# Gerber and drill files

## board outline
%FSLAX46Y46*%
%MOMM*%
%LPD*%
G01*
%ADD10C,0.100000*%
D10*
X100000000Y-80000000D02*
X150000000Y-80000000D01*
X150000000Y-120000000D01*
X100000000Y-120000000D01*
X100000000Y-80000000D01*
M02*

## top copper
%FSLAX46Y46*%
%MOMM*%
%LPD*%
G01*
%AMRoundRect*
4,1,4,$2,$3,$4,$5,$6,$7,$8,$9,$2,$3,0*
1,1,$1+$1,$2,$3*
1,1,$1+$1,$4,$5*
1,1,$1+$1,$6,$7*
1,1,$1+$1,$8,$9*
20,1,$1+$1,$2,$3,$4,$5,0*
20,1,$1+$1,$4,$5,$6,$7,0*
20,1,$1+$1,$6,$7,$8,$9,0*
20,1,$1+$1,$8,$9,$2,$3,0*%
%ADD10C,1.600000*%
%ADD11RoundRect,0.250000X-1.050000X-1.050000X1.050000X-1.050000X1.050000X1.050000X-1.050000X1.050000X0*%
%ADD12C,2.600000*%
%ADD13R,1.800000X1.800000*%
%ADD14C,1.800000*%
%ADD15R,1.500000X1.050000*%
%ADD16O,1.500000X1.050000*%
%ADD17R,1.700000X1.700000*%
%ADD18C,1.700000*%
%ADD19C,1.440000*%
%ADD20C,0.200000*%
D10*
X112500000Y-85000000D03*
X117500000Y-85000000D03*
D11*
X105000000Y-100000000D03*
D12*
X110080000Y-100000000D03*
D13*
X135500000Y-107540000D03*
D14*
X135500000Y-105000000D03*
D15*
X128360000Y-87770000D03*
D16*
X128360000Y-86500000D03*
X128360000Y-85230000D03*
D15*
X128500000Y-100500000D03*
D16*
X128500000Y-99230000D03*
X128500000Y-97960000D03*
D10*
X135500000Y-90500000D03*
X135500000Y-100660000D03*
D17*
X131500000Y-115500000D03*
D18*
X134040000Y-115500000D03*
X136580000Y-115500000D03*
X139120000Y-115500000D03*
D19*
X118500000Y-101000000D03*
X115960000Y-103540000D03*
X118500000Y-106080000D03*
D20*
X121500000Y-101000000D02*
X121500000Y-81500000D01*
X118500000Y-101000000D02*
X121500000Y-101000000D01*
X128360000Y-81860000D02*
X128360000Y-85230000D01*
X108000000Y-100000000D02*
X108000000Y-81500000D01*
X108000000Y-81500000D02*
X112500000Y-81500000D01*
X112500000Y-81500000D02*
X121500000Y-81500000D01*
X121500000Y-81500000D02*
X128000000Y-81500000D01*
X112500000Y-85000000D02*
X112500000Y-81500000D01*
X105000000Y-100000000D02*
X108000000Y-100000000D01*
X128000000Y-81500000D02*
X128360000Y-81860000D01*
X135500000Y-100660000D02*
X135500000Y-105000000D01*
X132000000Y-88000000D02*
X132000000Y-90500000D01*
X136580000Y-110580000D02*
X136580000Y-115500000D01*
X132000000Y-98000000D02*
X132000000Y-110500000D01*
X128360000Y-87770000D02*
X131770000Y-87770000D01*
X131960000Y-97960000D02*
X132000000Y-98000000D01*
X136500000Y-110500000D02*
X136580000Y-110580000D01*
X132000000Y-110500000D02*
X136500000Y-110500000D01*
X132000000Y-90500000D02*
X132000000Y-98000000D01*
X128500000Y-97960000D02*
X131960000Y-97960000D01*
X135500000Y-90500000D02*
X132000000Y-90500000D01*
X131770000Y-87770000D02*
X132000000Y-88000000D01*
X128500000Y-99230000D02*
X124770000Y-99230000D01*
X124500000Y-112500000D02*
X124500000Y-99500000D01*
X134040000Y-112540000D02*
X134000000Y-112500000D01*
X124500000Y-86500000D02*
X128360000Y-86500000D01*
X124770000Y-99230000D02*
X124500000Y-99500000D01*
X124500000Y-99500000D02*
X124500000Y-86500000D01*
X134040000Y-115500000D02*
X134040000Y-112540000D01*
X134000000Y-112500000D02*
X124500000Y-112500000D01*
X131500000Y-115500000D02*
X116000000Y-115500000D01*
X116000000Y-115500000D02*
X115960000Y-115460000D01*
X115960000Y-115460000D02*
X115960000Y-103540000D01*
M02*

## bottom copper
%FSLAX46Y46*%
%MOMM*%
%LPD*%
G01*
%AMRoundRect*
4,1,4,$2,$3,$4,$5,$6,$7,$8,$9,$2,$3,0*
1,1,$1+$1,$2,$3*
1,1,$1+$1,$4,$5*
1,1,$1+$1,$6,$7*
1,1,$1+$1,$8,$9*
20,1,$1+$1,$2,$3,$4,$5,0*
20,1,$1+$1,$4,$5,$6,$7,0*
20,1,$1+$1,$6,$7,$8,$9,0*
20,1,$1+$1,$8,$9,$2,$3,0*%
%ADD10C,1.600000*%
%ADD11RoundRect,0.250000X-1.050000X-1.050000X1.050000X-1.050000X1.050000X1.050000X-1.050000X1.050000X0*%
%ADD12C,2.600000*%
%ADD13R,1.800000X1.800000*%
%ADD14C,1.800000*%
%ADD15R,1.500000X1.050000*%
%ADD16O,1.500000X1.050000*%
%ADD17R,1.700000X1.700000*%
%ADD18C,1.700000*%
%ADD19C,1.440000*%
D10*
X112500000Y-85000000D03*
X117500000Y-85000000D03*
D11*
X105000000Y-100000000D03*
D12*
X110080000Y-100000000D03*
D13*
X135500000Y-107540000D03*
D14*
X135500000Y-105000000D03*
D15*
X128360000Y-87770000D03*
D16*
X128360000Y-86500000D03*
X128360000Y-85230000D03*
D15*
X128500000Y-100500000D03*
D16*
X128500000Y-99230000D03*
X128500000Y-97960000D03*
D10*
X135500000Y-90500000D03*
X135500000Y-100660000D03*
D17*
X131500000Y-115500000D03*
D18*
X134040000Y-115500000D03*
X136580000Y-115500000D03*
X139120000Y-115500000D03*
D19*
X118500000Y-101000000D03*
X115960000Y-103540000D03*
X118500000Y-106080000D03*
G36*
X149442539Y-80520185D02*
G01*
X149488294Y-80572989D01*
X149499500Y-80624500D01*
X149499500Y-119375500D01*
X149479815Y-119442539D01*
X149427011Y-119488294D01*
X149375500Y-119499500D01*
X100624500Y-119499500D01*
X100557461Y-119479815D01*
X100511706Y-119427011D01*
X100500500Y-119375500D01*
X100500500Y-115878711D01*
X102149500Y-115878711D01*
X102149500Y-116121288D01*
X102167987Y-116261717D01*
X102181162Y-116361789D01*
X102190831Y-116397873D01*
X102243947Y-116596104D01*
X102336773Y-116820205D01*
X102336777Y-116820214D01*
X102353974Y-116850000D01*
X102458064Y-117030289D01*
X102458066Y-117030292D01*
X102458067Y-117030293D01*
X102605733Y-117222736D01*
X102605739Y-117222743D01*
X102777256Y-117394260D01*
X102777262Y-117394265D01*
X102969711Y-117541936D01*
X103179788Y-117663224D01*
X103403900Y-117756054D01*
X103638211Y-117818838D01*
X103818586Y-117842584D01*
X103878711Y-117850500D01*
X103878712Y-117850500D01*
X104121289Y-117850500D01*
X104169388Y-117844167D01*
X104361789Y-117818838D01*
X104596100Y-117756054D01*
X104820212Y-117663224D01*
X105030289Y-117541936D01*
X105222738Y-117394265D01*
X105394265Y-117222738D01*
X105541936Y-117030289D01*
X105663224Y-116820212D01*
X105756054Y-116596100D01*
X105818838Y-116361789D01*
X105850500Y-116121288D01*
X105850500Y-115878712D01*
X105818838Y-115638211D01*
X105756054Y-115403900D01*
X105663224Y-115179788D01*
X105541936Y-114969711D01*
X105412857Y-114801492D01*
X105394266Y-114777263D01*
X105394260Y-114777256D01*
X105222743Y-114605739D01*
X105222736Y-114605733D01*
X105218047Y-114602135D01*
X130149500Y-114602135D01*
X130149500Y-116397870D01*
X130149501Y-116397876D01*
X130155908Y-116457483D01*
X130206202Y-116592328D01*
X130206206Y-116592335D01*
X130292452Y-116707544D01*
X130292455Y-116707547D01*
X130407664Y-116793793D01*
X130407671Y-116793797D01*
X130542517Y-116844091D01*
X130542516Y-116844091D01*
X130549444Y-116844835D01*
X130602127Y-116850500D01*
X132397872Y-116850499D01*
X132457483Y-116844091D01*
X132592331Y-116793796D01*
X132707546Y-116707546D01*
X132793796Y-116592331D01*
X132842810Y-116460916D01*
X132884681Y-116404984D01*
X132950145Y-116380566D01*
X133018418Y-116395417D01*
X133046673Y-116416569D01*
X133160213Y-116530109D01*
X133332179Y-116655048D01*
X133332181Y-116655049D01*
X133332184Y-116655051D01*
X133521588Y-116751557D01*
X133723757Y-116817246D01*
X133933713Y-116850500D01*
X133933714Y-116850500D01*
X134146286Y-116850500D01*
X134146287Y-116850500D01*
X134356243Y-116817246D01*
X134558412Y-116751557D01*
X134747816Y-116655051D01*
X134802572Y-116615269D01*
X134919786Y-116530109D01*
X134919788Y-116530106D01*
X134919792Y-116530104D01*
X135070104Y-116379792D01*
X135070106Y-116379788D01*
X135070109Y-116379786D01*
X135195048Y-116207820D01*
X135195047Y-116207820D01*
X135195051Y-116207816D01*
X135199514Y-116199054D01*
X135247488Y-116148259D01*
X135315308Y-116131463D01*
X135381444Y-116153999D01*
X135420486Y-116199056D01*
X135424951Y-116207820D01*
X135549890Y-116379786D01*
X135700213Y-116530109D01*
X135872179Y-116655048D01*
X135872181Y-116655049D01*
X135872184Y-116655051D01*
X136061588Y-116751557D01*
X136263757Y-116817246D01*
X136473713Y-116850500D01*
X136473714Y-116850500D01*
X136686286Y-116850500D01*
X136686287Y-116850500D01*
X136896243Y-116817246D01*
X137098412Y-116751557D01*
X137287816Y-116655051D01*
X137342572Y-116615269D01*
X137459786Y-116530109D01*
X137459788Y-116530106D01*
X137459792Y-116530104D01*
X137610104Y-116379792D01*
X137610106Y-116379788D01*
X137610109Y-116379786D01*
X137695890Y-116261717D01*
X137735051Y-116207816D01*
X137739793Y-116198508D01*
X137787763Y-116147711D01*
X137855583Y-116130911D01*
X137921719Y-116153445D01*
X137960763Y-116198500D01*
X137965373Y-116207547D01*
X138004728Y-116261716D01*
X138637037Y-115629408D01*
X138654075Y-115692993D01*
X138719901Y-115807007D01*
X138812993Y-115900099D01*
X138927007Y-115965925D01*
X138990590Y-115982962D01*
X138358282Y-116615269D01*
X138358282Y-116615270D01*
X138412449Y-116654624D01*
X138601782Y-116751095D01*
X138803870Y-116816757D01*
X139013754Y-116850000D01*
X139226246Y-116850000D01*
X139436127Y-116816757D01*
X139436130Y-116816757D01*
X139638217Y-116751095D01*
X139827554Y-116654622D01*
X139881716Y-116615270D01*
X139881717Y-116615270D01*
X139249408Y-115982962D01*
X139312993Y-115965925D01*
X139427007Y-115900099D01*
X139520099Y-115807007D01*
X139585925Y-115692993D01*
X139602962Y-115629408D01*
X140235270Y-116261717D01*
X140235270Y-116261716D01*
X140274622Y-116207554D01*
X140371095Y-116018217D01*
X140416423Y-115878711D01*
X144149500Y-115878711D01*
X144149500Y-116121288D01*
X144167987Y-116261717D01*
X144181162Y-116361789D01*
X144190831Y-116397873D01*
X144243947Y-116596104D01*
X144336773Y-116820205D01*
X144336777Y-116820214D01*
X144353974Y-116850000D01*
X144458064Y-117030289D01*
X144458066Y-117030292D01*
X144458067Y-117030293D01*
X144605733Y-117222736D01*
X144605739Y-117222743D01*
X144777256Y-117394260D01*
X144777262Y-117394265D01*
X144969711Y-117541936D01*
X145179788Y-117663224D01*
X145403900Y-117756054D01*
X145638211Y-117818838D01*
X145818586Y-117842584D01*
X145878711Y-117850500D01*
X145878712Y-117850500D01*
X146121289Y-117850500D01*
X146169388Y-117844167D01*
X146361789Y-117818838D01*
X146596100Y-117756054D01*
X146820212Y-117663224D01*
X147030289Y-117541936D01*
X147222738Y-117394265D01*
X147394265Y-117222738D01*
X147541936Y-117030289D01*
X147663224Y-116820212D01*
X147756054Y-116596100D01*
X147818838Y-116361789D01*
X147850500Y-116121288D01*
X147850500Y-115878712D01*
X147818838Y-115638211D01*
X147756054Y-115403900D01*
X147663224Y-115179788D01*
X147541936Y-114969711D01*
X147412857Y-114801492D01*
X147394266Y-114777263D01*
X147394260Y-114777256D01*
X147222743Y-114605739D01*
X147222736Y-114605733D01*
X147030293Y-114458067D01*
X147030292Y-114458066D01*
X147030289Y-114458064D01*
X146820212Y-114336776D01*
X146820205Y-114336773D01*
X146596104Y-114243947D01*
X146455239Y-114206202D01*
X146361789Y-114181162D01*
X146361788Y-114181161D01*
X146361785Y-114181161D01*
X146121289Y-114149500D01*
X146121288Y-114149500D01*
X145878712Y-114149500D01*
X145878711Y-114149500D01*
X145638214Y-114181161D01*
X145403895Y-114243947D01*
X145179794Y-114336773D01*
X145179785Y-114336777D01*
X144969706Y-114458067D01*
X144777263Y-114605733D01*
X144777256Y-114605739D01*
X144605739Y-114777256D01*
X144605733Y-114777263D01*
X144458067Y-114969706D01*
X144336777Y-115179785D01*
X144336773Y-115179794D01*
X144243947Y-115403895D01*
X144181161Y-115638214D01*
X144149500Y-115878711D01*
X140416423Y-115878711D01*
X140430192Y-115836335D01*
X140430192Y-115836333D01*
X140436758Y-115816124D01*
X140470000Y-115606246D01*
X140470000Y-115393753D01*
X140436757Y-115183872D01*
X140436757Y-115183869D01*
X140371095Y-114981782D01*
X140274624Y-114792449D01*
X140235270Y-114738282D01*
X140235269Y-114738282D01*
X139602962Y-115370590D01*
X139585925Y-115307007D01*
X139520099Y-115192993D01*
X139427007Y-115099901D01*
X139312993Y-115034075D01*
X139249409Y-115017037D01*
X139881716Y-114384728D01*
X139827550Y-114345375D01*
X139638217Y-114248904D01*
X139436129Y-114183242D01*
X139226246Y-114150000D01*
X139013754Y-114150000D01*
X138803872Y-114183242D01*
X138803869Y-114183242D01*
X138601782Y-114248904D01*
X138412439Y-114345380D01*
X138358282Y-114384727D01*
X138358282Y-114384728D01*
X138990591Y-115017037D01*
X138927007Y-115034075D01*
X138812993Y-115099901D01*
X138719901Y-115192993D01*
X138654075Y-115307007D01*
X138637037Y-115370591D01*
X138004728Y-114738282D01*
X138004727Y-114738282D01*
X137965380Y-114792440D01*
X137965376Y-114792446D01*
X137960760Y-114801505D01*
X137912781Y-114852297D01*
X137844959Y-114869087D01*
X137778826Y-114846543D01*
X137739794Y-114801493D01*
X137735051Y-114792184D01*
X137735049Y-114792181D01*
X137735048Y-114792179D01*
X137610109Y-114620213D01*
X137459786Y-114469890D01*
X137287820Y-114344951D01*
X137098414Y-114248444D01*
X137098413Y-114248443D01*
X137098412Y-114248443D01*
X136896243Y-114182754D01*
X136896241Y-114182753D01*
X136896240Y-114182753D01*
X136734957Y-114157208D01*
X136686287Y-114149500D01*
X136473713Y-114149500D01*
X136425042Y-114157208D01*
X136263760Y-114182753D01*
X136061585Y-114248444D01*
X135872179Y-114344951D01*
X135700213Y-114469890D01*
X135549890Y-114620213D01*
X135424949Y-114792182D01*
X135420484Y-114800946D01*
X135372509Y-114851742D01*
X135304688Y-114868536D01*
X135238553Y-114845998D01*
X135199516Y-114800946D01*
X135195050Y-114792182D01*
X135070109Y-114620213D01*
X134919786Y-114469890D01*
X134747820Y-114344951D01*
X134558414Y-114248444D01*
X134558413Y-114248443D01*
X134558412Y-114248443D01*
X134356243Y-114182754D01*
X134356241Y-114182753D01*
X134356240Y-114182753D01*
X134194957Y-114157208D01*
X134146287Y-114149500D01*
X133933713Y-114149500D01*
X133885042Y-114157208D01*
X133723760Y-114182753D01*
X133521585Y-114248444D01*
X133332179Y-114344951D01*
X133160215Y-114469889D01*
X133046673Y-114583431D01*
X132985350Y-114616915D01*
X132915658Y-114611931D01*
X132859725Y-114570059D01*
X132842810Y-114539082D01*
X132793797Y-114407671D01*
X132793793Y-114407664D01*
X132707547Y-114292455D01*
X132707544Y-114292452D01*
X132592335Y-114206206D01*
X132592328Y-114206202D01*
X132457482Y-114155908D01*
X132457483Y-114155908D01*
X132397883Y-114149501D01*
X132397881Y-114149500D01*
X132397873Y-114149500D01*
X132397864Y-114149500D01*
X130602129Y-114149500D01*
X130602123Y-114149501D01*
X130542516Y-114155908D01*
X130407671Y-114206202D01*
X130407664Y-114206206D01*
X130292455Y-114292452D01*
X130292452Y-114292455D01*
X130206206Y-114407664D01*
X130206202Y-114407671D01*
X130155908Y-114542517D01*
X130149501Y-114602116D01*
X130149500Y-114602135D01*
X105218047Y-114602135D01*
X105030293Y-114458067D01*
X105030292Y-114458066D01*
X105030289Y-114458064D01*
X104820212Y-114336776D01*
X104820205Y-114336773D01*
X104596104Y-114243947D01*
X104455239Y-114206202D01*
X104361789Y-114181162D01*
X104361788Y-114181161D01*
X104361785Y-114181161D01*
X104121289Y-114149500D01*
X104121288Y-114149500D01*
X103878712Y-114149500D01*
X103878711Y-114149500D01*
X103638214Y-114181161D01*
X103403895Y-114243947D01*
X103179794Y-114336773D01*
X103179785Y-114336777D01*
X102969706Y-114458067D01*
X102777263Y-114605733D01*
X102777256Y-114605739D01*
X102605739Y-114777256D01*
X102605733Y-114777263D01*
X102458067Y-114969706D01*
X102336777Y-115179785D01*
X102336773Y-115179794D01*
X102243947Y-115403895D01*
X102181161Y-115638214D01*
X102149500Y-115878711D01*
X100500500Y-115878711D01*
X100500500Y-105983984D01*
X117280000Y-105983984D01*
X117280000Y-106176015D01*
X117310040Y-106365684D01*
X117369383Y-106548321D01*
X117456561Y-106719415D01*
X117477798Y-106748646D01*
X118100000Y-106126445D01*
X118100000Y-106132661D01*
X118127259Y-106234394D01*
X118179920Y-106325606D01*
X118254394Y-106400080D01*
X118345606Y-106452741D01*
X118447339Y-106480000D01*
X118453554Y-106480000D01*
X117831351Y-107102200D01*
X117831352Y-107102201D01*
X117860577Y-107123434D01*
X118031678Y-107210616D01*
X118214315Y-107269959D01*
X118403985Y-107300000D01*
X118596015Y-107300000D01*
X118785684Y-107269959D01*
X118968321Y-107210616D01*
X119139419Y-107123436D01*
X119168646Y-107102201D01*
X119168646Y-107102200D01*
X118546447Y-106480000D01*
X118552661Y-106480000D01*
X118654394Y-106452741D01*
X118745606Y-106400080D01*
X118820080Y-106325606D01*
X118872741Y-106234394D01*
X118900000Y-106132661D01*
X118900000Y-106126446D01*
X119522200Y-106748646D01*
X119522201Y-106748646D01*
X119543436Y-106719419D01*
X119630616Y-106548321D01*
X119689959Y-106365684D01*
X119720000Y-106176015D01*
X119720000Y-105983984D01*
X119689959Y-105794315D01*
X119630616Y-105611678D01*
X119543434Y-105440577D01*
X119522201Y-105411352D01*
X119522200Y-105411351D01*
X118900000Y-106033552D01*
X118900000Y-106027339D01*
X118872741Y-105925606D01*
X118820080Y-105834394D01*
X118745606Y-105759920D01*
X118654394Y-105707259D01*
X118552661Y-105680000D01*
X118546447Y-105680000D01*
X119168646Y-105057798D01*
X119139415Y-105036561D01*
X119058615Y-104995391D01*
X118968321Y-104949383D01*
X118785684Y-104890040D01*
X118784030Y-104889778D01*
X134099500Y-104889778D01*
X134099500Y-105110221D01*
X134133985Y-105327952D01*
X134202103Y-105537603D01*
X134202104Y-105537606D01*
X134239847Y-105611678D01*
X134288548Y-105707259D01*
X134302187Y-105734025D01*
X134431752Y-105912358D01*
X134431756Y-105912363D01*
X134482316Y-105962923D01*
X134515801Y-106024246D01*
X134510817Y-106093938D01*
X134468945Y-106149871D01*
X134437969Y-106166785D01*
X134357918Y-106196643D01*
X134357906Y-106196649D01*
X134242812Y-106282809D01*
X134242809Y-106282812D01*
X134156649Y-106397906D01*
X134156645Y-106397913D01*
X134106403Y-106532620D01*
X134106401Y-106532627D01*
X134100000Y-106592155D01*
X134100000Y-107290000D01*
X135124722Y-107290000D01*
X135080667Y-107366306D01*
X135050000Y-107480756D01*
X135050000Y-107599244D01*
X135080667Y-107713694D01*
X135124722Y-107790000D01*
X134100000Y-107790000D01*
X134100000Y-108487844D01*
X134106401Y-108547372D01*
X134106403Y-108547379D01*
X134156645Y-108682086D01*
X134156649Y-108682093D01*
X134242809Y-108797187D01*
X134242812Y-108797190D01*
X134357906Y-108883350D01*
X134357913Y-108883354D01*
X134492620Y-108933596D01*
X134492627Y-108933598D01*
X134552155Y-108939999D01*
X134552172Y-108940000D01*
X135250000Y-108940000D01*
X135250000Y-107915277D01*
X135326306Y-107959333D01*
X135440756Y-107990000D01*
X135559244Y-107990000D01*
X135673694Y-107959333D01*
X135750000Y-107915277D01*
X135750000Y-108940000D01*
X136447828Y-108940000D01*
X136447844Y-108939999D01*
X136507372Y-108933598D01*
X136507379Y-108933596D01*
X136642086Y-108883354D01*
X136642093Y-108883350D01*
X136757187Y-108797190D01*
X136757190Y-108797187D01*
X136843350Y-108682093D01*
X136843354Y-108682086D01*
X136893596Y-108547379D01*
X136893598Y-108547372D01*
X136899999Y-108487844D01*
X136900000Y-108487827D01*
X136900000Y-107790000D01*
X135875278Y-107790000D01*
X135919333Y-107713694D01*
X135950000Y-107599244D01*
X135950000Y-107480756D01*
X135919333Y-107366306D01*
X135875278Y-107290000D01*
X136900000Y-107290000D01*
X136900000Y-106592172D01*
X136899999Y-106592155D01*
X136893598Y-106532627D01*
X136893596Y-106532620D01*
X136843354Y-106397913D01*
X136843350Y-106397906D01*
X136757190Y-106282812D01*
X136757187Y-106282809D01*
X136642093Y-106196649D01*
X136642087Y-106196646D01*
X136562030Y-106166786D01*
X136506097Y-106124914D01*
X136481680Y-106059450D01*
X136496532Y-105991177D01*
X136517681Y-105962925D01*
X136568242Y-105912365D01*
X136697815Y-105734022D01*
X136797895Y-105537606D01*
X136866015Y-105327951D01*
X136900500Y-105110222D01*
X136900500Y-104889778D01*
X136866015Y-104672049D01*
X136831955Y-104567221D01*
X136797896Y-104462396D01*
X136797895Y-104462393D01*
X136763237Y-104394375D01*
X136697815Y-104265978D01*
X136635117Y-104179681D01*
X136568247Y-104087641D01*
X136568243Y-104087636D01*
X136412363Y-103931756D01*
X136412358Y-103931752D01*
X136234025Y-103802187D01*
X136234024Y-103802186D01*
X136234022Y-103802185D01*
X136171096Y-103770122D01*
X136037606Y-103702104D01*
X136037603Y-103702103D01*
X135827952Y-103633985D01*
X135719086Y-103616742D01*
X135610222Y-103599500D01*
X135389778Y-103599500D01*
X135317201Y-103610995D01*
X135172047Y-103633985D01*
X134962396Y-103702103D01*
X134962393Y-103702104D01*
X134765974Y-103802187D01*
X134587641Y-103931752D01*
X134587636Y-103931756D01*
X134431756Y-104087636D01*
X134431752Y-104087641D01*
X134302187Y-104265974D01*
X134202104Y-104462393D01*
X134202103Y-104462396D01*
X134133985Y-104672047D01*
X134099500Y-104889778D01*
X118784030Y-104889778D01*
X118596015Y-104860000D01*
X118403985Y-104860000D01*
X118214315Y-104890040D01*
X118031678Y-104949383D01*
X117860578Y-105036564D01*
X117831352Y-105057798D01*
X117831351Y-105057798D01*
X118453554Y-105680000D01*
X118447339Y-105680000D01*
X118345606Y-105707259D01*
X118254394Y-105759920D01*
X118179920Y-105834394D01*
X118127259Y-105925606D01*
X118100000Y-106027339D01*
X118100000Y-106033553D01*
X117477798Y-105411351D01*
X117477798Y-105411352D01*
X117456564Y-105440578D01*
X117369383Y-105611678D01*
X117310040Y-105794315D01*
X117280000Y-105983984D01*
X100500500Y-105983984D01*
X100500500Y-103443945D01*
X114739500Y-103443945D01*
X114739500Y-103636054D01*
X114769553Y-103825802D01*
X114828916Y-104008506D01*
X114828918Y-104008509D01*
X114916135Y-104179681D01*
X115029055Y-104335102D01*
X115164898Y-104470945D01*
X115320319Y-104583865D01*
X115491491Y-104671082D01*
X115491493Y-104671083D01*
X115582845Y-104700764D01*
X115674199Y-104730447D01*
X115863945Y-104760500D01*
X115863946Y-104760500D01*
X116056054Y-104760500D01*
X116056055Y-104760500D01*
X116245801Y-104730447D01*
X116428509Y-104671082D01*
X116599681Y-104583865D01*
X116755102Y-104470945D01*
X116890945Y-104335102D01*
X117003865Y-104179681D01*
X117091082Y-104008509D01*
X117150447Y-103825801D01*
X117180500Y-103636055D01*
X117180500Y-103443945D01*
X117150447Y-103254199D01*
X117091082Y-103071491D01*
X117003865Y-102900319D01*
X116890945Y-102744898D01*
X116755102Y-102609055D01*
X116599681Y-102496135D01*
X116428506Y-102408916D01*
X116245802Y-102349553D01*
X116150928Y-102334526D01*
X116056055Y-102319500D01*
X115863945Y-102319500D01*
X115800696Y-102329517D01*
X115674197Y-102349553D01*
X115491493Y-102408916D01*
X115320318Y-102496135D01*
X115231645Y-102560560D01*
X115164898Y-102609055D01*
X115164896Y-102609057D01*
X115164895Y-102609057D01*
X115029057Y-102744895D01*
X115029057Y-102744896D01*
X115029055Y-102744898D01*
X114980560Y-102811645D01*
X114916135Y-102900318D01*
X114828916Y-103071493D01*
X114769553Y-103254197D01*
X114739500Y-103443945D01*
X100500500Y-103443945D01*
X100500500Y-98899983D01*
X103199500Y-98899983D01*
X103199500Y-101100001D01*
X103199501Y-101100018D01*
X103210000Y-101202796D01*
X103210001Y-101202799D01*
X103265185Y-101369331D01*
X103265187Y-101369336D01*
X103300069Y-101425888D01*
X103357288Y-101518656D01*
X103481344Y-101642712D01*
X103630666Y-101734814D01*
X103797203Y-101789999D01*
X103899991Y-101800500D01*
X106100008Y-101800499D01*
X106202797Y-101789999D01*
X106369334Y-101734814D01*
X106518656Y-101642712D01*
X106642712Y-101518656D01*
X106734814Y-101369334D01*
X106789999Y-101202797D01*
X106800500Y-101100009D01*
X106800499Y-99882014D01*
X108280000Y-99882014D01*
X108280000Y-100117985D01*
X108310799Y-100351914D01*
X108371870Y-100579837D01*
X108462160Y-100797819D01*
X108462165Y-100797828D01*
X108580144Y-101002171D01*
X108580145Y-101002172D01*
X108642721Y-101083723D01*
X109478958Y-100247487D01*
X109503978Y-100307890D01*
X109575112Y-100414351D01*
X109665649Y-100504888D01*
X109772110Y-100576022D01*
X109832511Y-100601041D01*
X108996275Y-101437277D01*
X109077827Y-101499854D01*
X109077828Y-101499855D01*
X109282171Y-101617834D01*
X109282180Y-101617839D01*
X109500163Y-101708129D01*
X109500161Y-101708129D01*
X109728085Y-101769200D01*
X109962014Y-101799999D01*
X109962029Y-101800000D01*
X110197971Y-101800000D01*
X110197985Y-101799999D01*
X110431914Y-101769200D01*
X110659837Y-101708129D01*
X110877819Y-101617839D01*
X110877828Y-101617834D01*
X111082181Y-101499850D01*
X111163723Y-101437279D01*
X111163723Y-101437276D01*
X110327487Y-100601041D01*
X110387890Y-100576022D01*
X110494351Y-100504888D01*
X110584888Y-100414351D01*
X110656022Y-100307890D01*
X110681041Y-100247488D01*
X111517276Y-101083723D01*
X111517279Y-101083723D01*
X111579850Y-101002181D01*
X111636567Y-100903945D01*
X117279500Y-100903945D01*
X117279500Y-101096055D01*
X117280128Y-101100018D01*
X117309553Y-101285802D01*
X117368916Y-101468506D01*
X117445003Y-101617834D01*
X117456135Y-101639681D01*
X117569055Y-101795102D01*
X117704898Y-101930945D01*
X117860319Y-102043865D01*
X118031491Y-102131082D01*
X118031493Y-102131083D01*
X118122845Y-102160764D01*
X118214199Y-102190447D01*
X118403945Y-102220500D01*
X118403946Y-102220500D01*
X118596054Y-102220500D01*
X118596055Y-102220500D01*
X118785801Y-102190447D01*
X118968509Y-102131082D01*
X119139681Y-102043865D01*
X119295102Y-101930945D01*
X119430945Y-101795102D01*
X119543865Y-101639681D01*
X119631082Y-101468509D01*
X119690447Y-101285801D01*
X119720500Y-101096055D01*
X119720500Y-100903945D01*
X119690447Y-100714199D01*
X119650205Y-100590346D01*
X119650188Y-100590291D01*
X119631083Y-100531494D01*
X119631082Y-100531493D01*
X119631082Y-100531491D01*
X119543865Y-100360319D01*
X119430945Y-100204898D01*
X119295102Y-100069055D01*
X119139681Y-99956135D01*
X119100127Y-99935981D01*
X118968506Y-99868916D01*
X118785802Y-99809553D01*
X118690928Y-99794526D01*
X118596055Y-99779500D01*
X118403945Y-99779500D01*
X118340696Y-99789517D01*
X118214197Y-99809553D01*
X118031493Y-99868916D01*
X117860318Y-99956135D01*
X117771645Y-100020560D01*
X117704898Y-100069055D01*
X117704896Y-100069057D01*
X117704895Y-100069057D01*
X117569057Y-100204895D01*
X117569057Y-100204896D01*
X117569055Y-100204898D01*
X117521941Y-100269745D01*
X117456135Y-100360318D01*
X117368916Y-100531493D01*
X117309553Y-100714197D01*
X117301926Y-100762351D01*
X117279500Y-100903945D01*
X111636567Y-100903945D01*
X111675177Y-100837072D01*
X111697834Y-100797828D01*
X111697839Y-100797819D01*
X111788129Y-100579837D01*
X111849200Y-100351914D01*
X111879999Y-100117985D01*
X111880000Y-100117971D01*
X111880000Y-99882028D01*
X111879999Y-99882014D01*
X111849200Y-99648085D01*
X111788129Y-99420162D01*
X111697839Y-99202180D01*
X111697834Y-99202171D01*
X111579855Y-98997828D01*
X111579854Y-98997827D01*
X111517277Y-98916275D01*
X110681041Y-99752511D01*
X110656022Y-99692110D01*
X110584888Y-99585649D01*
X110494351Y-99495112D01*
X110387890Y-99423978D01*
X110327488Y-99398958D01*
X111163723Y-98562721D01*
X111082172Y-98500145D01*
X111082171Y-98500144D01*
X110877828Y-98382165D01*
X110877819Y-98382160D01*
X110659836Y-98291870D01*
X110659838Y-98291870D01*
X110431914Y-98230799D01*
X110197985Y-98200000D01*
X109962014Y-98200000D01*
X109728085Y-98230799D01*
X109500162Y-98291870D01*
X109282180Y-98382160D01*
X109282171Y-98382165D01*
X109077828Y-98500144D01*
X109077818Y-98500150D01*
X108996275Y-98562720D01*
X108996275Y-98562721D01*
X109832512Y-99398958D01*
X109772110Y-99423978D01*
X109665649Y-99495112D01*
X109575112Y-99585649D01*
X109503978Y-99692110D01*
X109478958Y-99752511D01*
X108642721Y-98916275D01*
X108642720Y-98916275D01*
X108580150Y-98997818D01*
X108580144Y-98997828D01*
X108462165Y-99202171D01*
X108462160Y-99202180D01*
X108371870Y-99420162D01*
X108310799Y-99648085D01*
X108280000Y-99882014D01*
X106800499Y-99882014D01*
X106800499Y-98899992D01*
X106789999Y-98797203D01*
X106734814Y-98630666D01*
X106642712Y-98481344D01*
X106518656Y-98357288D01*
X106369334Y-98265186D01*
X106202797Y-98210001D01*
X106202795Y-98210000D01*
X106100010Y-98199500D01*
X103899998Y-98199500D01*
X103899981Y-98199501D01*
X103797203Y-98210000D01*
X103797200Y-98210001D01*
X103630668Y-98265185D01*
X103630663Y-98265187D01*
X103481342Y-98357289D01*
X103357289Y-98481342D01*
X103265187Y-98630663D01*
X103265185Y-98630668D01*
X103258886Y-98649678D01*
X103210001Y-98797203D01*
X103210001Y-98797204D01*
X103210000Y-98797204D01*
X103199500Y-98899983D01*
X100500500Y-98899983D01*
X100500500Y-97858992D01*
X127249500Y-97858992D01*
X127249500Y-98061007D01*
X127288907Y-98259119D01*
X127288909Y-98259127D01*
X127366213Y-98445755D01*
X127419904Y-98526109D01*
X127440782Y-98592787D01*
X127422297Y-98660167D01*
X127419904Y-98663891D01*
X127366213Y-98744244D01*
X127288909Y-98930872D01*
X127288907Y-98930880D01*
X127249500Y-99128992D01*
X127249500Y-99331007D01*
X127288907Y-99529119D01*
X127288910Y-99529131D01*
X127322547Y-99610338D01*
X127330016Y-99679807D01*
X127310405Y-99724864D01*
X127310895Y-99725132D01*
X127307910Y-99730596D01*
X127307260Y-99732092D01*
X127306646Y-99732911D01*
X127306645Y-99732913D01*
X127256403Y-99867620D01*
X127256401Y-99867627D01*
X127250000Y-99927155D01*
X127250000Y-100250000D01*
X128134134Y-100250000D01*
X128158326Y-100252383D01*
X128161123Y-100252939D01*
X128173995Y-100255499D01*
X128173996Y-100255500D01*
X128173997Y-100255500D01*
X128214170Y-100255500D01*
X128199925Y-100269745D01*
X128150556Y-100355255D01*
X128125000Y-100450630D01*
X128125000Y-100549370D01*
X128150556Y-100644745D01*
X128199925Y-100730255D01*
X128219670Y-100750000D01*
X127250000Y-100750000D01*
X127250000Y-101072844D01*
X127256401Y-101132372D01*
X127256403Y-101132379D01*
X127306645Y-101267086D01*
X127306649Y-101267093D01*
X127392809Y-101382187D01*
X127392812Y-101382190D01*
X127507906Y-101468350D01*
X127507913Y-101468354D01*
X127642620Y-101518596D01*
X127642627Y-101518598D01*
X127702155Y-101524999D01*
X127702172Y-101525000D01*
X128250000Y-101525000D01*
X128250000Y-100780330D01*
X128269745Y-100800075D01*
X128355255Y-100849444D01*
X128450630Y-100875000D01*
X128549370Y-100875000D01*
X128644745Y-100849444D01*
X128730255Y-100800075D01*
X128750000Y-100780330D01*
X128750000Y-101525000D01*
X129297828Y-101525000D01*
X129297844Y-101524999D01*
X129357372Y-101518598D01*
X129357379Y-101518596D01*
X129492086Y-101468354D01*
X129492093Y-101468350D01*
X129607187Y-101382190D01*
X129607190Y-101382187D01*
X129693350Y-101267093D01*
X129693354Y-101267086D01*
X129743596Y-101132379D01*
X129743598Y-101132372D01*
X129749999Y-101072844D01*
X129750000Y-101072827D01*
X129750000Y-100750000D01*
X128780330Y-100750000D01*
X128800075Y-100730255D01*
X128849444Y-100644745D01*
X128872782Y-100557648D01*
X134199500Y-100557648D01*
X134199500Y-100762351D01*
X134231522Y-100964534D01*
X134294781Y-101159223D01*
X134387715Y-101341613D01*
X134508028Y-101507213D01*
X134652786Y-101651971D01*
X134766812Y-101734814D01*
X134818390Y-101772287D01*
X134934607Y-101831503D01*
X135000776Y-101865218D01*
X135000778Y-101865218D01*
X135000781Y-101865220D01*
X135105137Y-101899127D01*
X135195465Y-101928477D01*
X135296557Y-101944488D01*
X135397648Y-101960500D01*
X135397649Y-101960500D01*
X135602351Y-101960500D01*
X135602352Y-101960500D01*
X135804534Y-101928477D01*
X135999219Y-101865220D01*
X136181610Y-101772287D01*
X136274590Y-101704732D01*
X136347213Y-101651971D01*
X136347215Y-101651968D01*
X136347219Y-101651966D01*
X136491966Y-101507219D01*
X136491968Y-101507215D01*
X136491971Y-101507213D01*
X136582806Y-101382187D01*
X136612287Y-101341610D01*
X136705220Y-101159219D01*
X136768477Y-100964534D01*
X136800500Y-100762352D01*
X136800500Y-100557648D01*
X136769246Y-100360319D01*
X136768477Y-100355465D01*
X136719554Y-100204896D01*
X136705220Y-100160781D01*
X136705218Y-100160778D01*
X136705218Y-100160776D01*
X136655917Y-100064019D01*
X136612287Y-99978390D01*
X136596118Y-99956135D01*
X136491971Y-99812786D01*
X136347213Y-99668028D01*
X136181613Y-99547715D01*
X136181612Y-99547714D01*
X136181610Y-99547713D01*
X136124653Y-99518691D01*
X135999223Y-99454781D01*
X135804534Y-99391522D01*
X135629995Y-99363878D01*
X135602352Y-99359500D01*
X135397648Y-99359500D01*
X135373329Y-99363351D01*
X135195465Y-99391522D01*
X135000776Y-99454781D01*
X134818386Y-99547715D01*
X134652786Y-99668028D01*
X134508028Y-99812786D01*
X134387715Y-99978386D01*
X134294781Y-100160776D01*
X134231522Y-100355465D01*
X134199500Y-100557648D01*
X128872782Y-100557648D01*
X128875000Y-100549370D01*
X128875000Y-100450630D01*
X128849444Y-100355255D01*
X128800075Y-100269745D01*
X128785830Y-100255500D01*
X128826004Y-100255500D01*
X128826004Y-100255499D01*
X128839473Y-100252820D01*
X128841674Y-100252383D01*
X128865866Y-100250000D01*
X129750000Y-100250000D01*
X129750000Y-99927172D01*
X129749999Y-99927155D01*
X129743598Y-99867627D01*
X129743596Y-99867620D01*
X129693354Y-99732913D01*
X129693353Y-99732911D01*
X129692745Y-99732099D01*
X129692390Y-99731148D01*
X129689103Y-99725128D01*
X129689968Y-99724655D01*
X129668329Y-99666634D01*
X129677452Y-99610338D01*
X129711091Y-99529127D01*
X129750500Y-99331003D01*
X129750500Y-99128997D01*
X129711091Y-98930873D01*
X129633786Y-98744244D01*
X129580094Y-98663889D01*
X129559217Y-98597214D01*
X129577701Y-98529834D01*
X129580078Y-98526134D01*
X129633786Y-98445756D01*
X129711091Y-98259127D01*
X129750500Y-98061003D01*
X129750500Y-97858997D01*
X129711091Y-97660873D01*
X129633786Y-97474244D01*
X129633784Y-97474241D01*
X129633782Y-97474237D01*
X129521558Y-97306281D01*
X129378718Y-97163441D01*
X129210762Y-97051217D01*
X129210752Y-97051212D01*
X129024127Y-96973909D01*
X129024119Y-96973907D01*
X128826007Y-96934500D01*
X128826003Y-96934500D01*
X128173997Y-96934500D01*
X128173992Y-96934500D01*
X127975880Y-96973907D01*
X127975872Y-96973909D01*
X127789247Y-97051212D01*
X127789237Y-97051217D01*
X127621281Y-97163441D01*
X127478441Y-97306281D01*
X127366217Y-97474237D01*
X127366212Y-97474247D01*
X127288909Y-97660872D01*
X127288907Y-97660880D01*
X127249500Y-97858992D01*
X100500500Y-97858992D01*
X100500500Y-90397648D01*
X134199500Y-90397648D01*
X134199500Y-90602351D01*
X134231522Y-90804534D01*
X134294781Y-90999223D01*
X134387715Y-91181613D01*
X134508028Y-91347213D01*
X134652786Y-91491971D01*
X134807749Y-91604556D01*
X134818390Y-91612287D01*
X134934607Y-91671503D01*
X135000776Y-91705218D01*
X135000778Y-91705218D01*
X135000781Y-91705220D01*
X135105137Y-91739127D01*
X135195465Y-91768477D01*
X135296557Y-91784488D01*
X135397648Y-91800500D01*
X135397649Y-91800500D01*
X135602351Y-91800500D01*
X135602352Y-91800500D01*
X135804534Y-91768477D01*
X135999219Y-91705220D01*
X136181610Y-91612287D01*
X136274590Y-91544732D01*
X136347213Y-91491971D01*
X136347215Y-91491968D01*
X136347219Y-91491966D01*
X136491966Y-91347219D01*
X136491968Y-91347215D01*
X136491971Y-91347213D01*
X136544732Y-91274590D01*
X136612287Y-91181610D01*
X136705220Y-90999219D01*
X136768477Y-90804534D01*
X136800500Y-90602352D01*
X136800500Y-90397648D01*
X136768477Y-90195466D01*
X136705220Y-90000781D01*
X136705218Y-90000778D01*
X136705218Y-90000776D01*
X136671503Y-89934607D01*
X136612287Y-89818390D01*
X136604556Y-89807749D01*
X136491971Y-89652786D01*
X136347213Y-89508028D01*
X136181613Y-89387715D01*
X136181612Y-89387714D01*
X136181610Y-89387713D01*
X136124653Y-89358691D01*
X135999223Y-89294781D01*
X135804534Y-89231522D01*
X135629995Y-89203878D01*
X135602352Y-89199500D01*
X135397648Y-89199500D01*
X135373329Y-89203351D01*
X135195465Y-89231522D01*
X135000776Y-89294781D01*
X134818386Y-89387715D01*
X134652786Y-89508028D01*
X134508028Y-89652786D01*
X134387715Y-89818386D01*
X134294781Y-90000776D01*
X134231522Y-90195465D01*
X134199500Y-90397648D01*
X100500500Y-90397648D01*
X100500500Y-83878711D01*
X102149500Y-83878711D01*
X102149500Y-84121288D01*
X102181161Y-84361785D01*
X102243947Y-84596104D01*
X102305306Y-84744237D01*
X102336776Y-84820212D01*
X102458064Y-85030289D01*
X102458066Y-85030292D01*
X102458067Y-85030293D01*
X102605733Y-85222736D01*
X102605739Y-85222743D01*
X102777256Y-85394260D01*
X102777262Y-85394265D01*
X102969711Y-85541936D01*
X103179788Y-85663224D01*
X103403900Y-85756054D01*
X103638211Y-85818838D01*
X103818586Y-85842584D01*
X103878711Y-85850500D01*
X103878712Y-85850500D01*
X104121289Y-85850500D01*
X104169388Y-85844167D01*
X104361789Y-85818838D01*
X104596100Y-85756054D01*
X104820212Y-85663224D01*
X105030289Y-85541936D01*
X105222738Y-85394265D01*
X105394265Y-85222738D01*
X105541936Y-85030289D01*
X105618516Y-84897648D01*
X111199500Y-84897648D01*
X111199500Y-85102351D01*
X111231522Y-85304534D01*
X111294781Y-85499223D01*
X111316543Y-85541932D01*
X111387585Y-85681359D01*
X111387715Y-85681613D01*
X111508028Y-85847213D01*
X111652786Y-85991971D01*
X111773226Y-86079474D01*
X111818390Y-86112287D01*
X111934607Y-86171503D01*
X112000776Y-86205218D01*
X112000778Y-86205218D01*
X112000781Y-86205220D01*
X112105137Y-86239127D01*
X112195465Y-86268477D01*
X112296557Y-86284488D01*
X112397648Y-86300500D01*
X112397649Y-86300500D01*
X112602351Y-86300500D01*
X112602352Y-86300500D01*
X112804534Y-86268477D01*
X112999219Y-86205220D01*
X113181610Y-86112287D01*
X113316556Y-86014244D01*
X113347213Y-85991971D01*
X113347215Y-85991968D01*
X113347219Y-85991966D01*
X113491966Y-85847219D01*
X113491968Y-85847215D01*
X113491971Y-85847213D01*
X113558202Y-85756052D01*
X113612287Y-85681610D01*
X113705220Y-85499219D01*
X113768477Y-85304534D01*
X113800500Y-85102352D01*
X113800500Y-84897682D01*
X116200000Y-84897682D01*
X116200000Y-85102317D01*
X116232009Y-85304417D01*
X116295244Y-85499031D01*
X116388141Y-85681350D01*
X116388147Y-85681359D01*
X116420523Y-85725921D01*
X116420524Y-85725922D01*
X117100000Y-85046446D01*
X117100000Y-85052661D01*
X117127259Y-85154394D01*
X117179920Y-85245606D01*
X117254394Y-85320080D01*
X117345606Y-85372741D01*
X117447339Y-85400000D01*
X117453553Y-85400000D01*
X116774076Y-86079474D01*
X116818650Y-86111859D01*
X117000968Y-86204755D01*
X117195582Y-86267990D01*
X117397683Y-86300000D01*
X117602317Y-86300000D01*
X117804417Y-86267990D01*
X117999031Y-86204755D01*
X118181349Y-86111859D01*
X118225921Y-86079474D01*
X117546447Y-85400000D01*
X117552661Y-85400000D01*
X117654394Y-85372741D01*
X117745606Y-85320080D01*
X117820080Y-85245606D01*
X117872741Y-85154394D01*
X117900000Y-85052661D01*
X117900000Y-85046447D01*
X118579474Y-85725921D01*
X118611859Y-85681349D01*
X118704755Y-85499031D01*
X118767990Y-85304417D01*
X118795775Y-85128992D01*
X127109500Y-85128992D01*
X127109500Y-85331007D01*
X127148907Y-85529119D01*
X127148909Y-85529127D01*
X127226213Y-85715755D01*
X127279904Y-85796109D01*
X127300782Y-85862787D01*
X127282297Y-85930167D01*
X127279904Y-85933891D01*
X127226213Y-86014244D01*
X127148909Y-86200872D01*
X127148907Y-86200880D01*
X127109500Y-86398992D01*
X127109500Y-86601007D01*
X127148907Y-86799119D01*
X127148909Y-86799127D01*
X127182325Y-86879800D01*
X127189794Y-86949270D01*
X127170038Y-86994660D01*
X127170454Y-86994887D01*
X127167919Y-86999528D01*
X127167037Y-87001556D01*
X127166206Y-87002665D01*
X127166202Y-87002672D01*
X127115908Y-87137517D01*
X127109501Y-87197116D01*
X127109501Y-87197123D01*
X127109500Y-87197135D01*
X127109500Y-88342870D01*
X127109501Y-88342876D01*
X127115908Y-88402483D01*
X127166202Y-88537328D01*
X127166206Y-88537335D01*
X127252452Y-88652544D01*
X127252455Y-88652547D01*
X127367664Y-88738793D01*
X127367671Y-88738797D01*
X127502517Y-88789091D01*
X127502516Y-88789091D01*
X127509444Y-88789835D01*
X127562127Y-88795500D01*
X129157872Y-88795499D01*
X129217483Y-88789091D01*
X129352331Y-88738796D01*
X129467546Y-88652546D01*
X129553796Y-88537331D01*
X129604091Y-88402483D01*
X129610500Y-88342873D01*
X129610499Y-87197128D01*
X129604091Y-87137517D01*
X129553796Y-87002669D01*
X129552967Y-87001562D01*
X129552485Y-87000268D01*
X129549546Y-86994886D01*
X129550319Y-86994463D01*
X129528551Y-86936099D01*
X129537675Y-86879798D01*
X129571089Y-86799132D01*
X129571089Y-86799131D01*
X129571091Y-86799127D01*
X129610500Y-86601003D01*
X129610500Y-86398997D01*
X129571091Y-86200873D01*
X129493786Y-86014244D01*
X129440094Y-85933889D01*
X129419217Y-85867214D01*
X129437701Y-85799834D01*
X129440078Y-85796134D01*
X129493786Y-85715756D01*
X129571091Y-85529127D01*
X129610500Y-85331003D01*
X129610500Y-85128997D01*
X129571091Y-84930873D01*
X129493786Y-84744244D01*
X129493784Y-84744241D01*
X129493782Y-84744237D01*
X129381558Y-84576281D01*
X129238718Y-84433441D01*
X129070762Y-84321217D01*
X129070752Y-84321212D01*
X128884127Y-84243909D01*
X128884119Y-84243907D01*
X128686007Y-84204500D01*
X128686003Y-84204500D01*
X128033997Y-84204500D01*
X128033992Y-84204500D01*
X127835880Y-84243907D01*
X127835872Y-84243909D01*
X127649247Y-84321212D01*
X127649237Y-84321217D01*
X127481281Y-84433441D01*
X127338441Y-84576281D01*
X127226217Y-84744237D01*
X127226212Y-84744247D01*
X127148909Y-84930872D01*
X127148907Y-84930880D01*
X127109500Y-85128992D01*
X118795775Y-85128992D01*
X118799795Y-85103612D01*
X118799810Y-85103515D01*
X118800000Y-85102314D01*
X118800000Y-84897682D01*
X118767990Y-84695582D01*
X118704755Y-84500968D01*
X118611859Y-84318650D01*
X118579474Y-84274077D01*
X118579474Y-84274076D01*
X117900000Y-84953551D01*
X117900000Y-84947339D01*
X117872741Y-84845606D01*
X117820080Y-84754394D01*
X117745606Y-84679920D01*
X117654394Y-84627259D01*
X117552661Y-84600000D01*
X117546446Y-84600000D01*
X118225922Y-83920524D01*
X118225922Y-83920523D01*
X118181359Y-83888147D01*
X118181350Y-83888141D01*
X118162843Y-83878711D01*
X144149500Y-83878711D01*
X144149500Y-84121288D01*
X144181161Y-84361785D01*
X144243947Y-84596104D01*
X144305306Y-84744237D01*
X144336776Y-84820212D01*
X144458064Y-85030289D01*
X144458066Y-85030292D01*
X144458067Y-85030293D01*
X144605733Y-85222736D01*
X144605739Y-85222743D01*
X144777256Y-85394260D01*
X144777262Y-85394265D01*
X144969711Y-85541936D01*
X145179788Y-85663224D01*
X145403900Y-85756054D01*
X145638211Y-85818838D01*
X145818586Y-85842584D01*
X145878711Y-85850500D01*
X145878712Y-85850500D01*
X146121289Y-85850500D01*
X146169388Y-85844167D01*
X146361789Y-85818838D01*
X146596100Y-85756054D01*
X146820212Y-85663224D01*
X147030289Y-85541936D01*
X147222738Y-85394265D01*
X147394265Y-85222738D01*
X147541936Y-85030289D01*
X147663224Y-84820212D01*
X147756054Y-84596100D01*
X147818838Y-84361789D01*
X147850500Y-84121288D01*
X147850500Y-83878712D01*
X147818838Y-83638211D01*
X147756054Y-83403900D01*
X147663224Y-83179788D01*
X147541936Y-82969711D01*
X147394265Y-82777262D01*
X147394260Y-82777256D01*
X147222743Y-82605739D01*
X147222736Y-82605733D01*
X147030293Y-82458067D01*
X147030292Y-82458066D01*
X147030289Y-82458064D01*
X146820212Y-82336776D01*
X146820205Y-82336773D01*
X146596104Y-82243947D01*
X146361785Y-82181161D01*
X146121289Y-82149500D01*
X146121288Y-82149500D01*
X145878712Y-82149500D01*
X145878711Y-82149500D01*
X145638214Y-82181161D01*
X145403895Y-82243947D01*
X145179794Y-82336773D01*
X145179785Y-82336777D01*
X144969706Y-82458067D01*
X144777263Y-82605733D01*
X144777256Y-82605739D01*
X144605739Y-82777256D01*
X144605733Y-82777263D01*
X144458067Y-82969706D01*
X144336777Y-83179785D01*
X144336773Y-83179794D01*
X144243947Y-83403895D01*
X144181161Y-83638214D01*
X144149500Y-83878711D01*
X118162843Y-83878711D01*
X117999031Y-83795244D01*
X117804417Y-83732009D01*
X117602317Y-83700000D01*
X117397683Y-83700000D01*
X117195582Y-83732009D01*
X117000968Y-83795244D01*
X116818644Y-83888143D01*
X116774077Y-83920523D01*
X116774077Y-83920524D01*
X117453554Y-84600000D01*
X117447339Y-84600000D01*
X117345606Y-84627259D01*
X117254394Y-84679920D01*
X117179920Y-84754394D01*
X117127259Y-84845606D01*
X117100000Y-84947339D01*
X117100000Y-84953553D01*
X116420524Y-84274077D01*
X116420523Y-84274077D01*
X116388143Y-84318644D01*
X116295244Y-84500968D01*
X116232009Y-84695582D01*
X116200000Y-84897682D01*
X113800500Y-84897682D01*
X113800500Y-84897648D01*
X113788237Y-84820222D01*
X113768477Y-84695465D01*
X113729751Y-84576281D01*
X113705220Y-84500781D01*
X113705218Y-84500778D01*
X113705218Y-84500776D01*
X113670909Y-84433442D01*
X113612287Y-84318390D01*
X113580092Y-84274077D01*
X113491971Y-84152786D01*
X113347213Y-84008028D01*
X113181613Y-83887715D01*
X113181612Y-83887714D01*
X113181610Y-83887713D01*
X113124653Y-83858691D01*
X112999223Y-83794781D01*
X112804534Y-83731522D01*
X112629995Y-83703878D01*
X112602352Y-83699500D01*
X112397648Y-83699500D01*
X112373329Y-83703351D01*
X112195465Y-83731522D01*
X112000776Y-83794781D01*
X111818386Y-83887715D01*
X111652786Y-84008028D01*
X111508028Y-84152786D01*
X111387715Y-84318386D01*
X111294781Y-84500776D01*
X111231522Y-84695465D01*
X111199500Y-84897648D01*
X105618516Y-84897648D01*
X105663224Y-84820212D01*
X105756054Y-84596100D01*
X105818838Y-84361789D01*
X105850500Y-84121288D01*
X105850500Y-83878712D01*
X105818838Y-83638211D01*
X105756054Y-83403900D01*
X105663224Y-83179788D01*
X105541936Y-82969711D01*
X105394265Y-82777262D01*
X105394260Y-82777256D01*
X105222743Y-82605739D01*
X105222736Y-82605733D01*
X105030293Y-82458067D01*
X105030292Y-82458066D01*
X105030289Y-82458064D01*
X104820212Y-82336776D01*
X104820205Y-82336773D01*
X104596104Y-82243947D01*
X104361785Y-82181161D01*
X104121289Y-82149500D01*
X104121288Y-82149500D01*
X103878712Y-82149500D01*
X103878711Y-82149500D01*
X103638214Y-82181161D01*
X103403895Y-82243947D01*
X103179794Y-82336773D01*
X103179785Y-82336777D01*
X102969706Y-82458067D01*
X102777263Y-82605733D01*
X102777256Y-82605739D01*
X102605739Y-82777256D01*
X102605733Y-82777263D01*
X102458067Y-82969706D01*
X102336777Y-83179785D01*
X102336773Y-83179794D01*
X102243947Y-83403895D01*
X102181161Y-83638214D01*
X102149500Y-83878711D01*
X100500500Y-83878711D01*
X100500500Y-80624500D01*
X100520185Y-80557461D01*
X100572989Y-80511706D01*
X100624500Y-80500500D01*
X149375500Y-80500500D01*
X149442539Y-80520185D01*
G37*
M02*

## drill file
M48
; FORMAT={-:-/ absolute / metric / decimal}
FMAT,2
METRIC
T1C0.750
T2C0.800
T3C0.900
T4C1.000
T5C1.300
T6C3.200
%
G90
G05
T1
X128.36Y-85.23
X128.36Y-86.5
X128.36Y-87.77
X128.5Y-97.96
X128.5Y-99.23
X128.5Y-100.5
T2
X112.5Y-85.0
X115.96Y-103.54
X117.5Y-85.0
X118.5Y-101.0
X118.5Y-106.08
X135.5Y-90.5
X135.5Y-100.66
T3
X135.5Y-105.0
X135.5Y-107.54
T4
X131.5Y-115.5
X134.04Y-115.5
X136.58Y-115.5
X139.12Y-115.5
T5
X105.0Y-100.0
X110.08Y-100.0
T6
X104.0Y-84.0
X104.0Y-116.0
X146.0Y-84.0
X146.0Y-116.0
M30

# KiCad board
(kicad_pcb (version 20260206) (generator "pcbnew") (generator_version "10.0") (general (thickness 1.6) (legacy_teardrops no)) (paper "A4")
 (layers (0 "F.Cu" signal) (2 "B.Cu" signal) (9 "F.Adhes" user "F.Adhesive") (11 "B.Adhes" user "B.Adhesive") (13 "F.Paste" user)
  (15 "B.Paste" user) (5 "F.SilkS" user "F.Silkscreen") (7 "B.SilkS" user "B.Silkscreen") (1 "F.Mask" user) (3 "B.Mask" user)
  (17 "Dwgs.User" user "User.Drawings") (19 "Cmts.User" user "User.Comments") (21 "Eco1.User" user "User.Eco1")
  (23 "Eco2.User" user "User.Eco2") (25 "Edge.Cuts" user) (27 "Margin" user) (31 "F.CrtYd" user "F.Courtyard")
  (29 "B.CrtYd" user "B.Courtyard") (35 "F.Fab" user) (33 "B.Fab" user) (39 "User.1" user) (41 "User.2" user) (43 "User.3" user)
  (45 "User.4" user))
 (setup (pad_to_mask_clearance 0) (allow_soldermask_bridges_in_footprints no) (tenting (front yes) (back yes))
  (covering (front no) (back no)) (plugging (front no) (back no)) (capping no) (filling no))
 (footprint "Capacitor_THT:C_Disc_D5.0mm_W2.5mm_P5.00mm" (layer "F.Cu") (at 112.5 85)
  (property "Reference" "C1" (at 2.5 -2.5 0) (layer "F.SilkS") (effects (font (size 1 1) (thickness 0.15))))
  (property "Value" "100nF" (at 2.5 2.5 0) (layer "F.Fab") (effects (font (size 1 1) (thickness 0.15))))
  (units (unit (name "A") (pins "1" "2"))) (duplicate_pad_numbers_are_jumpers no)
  (pad "1" thru_hole circle (at 0 0) (size 1.6 1.6) (drill 0.8) (layers "*.Cu" "*.Mask") (remove_unused_layers no) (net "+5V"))
  (pad "2" thru_hole circle (at 5 0) (size 1.6 1.6) (drill 0.8) (layers "*.Cu" "*.Mask") (remove_unused_layers no) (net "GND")))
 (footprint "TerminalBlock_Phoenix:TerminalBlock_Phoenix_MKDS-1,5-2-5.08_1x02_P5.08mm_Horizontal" (layer "F.Cu") (at 105 100)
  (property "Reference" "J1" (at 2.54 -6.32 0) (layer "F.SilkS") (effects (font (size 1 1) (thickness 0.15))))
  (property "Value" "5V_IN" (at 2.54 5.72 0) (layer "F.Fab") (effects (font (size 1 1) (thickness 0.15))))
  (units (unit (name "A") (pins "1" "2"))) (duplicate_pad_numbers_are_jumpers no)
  (pad "1" thru_hole roundrect (at 0 0) (size 2.6 2.6) (drill 1.3) (layers "*.Cu" "*.Mask") (remove_unused_layers no)
   (roundrect_rratio 0.096154) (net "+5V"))
  (pad "2" thru_hole circle (at 5.08 0) (size 2.6 2.6) (drill 1.3) (layers "*.Cu" "*.Mask") (remove_unused_layers no) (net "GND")))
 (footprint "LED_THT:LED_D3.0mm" (layer "F.Cu") (at 135.5 107.54 90)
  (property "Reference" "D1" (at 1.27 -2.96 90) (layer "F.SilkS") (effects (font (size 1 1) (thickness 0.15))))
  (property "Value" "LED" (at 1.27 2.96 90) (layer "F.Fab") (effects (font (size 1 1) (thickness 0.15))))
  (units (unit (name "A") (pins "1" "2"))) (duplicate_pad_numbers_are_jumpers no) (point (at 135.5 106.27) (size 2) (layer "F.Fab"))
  (pad "1" thru_hole rect (at 0 0 90) (size 1.8 1.8) (drill 0.9) (layers "*.Cu" "*.Mask") (remove_unused_layers no) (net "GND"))
  (pad "2" thru_hole circle (at 2.54 0 90) (size 1.8 1.8) (drill 0.9) (layers "*.Cu" "*.Mask") (remove_unused_layers no) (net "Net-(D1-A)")))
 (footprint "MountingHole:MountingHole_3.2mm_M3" (layer "F.Cu") (at 104 116)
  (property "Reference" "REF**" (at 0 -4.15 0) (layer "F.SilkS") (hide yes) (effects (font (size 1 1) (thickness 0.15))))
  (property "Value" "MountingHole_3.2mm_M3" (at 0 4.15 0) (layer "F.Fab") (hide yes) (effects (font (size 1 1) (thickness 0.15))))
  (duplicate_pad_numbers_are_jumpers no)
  (pad "" np_thru_hole circle (at 0 0) (size 3.2 3.2) (drill 3.2) (layers "*.Cu" "*.Mask")))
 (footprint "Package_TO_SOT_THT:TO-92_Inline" (layer "F.Cu") (at 128.36 87.77 90)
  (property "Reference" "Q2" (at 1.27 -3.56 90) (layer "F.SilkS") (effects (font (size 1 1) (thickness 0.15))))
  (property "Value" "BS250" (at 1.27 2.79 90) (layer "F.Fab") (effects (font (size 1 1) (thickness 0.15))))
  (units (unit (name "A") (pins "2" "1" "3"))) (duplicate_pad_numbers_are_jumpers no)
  (pad "1" thru_hole rect (at 0 0 90) (size 1.05 1.5) (drill 0.75) (layers "*.Cu" "*.Mask") (remove_unused_layers no) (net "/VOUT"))
  (pad "2" thru_hole oval (at 1.27 0 90) (size 1.05 1.5) (drill 0.75) (layers "*.Cu" "*.Mask") (remove_unused_layers no) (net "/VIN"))
  (pad "3" thru_hole oval (at 2.54 0 90) (size 1.05 1.5) (drill 0.75) (layers "*.Cu" "*.Mask") (remove_unused_layers no) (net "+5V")))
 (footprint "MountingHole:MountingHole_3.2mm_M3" (layer "F.Cu") (at 146 84)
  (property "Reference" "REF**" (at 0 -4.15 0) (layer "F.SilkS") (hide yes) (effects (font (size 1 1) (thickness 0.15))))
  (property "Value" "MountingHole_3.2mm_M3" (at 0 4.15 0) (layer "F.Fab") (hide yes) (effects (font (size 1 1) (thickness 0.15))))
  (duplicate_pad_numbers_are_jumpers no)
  (pad "" np_thru_hole circle (at 0 0) (size 3.2 3.2) (drill 3.2) (layers "*.Cu" "*.Mask")))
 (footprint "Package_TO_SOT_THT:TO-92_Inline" (layer "F.Cu") (at 128.5 100.5 90)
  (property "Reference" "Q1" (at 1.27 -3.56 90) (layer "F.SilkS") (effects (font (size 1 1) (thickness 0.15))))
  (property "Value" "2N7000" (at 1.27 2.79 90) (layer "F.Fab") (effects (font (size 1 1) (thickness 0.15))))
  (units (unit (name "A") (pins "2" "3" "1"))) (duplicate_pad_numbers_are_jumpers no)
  (pad "1" thru_hole rect (at 0 0 90) (size 1.05 1.5) (drill 0.75) (layers "*.Cu" "*.Mask") (remove_unused_layers no) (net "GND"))
  (pad "2" thru_hole oval (at 1.27 0 90) (size 1.05 1.5) (drill 0.75) (layers "*.Cu" "*.Mask") (remove_unused_layers no) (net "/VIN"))
  (pad "3" thru_hole oval (at 2.54 0 90) (size 1.05 1.5) (drill 0.75) (layers "*.Cu" "*.Mask") (remove_unused_layers no) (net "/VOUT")))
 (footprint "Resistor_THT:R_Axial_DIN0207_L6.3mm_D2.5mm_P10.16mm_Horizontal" (layer "F.Cu") (at 135.5 90.5 -90)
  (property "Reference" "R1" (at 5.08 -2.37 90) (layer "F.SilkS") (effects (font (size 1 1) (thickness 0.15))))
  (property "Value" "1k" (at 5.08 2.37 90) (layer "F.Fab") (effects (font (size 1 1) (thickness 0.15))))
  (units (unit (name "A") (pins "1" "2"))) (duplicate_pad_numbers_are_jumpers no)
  (pad "1" thru_hole circle (at 0 0 270) (size 1.6 1.6) (drill 0.8) (layers "*.Cu" "*.Mask") (remove_unused_layers no) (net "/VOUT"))
  (pad "2" thru_hole circle (at 10.16 0 270) (size 1.6 1.6) (drill 0.8) (layers "*.Cu" "*.Mask") (remove_unused_layers no)
   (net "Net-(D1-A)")))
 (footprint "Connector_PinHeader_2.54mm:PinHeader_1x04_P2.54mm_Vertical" (layer "F.Cu") (at 131.5 115.5 90)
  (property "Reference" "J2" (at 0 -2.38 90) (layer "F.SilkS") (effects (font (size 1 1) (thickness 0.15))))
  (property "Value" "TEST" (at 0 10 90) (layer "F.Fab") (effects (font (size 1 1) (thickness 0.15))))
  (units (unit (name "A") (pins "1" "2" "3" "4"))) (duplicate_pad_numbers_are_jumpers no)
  (pad "1" thru_hole rect (at 0 0 90) (size 1.7 1.7) (drill 1) (layers "*.Cu" "*.Mask") (remove_unused_layers no) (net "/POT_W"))
  (pad "2" thru_hole circle (at 0 2.54 90) (size 1.7 1.7) (drill 1) (layers "*.Cu" "*.Mask") (remove_unused_layers no) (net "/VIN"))
  (pad "3" thru_hole circle (at 0 5.08 90) (size 1.7 1.7) (drill 1) (layers "*.Cu" "*.Mask") (remove_unused_layers no) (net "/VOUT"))
  (pad "4" thru_hole circle (at 0 7.62 90) (size 1.7 1.7) (drill 1) (layers "*.Cu" "*.Mask") (remove_unused_layers no) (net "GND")))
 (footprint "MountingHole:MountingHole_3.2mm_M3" (layer "F.Cu") (at 104 84)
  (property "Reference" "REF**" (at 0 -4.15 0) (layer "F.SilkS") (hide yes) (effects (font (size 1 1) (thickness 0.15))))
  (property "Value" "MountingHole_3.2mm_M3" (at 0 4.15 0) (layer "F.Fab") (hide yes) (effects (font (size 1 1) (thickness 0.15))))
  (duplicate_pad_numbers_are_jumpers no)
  (pad "" np_thru_hole circle (at 0 0) (size 3.2 3.2) (drill 3.2) (layers "*.Cu" "*.Mask")))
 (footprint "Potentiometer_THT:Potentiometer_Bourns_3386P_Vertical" (layer "F.Cu") (at 118.5 101 180)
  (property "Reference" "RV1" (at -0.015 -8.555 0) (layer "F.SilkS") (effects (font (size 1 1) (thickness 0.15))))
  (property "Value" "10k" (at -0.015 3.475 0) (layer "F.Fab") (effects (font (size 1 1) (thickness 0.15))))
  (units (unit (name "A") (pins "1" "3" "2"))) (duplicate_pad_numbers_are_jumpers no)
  (pad "1" thru_hole circle (at 0 0 180) (size 1.44 1.44) (drill 0.8) (layers "*.Cu" "*.Mask") (remove_unused_layers no) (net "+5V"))
  (pad "2" thru_hole circle (at 2.54 -2.54 180) (size 1.44 1.44) (drill 0.8) (layers "*.Cu" "*.Mask") (remove_unused_layers no)
   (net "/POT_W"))
  (pad "3" thru_hole circle (at 0 -5.08 180) (size 1.44 1.44) (drill 0.8) (layers "*.Cu" "*.Mask") (remove_unused_layers no) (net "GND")))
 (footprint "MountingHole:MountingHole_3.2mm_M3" (layer "F.Cu") (at 146 116)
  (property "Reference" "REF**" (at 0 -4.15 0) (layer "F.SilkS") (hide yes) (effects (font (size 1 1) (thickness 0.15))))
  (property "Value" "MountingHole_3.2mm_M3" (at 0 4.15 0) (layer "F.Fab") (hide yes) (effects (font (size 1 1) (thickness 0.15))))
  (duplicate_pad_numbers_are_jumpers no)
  (pad "" np_thru_hole circle (at 0 0) (size 3.2 3.2) (drill 3.2) (layers "*.Cu" "*.Mask")))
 (gr_rect (start 100 80) (end 150 120) (stroke (width 0.1) (type solid)) (fill no) (layer "Edge.Cuts"))
 (segment (start 121.5 101) (end 121.5 81.5) (width 0.2) (layer "F.Cu") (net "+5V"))
 (segment (start 118.5 101) (end 121.5 101) (width 0.2) (layer "F.Cu") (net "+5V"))
 (segment (start 128.36 81.86) (end 128.36 85.23) (width 0.2) (layer "F.Cu") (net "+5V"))
 (segment (start 108 100) (end 108 81.5) (width 0.2) (layer "F.Cu") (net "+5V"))
 (segment (start 108 81.5) (end 112.5 81.5) (width 0.2) (layer "F.Cu") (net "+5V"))
 (segment (start 112.5 81.5) (end 121.5 81.5) (width 0.2) (layer "F.Cu") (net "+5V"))
 (segment (start 121.5 81.5) (end 128 81.5) (width 0.2) (layer "F.Cu") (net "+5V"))
 (segment (start 112.5 85) (end 112.5 81.5) (width 0.2) (layer "F.Cu") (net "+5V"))
 (segment (start 105 100) (end 108 100) (width 0.2) (layer "F.Cu") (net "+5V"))
 (segment (start 128 81.5) (end 128.36 81.86) (width 0.2) (layer "F.Cu") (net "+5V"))
 (segment (start 135.5 100.66) (end 135.5 105) (width 0.2) (layer "F.Cu") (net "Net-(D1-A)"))
 (segment (start 132 88) (end 132 90.5) (width 0.2) (layer "F.Cu") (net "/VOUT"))
 (segment (start 136.58 110.58) (end 136.58 115.5) (width 0.2) (layer "F.Cu") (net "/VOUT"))
 (segment (start 132 98) (end 132 110.5) (width 0.2) (layer "F.Cu") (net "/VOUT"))
 (segment (start 128.36 87.77) (end 131.77 87.77) (width 0.2) (layer "F.Cu") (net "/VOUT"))
 (segment (start 131.96 97.96) (end 132 98) (width 0.2) (layer "F.Cu") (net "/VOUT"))
 (segment (start 136.5 110.5) (end 136.58 110.58) (width 0.2) (layer "F.Cu") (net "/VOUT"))
 (segment (start 132 110.5) (end 136.5 110.5) (width 0.2) (layer "F.Cu") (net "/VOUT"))
 (segment (start 132 90.5) (end 132 98) (width 0.2) (layer "F.Cu") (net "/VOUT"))
 (segment (start 128.5 97.96) (end 131.96 97.96) (width 0.2) (layer "F.Cu") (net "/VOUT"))
 (segment (start 135.5 90.5) (end 132 90.5) (width 0.2) (layer "F.Cu") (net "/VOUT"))
 (segment (start 131.77 87.77) (end 132 88) (width 0.2) (layer "F.Cu") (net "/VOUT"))
 (segment (start 128.5 99.23) (end 124.77 99.23) (width 0.2) (layer "F.Cu") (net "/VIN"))
 (segment (start 124.5 112.5) (end 124.5 99.5) (width 0.2) (layer "F.Cu") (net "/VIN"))
 (segment (start 134.04 112.54) (end 134 112.5) (width 0.2) (layer "F.Cu") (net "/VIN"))
 (segment (start 124.5 86.5) (end 128.36 86.5) (width 0.2) (layer "F.Cu") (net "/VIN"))
 (segment (start 124.77 99.23) (end 124.5 99.5) (width 0.2) (layer "F.Cu") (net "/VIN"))
 (segment (start 124.5 99.5) (end 124.5 86.5) (width 0.2) (layer "F.Cu") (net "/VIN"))
 (segment (start 134.04 115.5) (end 134.04 112.54) (width 0.2) (layer "F.Cu") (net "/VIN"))
 (segment (start 134 112.5) (end 124.5 112.5) (width 0.2) (layer "F.Cu") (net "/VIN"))
 (segment (start 131.5 115.5) (end 116 115.5) (width 0.2) (layer "F.Cu") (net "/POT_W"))
 (segment (start 116 115.5) (end 115.96 115.46) (width 0.2) (layer "F.Cu") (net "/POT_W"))
 (segment (start 115.96 115.46) (end 115.96 103.54) (width 0.2) (layer "F.Cu") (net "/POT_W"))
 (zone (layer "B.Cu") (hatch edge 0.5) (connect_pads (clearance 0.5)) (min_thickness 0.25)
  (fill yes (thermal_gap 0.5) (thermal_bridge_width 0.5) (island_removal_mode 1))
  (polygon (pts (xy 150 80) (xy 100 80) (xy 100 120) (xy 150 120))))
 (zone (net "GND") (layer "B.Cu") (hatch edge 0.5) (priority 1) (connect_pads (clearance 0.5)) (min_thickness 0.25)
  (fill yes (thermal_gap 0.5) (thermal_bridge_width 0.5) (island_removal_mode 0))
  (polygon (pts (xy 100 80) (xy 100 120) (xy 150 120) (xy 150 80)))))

